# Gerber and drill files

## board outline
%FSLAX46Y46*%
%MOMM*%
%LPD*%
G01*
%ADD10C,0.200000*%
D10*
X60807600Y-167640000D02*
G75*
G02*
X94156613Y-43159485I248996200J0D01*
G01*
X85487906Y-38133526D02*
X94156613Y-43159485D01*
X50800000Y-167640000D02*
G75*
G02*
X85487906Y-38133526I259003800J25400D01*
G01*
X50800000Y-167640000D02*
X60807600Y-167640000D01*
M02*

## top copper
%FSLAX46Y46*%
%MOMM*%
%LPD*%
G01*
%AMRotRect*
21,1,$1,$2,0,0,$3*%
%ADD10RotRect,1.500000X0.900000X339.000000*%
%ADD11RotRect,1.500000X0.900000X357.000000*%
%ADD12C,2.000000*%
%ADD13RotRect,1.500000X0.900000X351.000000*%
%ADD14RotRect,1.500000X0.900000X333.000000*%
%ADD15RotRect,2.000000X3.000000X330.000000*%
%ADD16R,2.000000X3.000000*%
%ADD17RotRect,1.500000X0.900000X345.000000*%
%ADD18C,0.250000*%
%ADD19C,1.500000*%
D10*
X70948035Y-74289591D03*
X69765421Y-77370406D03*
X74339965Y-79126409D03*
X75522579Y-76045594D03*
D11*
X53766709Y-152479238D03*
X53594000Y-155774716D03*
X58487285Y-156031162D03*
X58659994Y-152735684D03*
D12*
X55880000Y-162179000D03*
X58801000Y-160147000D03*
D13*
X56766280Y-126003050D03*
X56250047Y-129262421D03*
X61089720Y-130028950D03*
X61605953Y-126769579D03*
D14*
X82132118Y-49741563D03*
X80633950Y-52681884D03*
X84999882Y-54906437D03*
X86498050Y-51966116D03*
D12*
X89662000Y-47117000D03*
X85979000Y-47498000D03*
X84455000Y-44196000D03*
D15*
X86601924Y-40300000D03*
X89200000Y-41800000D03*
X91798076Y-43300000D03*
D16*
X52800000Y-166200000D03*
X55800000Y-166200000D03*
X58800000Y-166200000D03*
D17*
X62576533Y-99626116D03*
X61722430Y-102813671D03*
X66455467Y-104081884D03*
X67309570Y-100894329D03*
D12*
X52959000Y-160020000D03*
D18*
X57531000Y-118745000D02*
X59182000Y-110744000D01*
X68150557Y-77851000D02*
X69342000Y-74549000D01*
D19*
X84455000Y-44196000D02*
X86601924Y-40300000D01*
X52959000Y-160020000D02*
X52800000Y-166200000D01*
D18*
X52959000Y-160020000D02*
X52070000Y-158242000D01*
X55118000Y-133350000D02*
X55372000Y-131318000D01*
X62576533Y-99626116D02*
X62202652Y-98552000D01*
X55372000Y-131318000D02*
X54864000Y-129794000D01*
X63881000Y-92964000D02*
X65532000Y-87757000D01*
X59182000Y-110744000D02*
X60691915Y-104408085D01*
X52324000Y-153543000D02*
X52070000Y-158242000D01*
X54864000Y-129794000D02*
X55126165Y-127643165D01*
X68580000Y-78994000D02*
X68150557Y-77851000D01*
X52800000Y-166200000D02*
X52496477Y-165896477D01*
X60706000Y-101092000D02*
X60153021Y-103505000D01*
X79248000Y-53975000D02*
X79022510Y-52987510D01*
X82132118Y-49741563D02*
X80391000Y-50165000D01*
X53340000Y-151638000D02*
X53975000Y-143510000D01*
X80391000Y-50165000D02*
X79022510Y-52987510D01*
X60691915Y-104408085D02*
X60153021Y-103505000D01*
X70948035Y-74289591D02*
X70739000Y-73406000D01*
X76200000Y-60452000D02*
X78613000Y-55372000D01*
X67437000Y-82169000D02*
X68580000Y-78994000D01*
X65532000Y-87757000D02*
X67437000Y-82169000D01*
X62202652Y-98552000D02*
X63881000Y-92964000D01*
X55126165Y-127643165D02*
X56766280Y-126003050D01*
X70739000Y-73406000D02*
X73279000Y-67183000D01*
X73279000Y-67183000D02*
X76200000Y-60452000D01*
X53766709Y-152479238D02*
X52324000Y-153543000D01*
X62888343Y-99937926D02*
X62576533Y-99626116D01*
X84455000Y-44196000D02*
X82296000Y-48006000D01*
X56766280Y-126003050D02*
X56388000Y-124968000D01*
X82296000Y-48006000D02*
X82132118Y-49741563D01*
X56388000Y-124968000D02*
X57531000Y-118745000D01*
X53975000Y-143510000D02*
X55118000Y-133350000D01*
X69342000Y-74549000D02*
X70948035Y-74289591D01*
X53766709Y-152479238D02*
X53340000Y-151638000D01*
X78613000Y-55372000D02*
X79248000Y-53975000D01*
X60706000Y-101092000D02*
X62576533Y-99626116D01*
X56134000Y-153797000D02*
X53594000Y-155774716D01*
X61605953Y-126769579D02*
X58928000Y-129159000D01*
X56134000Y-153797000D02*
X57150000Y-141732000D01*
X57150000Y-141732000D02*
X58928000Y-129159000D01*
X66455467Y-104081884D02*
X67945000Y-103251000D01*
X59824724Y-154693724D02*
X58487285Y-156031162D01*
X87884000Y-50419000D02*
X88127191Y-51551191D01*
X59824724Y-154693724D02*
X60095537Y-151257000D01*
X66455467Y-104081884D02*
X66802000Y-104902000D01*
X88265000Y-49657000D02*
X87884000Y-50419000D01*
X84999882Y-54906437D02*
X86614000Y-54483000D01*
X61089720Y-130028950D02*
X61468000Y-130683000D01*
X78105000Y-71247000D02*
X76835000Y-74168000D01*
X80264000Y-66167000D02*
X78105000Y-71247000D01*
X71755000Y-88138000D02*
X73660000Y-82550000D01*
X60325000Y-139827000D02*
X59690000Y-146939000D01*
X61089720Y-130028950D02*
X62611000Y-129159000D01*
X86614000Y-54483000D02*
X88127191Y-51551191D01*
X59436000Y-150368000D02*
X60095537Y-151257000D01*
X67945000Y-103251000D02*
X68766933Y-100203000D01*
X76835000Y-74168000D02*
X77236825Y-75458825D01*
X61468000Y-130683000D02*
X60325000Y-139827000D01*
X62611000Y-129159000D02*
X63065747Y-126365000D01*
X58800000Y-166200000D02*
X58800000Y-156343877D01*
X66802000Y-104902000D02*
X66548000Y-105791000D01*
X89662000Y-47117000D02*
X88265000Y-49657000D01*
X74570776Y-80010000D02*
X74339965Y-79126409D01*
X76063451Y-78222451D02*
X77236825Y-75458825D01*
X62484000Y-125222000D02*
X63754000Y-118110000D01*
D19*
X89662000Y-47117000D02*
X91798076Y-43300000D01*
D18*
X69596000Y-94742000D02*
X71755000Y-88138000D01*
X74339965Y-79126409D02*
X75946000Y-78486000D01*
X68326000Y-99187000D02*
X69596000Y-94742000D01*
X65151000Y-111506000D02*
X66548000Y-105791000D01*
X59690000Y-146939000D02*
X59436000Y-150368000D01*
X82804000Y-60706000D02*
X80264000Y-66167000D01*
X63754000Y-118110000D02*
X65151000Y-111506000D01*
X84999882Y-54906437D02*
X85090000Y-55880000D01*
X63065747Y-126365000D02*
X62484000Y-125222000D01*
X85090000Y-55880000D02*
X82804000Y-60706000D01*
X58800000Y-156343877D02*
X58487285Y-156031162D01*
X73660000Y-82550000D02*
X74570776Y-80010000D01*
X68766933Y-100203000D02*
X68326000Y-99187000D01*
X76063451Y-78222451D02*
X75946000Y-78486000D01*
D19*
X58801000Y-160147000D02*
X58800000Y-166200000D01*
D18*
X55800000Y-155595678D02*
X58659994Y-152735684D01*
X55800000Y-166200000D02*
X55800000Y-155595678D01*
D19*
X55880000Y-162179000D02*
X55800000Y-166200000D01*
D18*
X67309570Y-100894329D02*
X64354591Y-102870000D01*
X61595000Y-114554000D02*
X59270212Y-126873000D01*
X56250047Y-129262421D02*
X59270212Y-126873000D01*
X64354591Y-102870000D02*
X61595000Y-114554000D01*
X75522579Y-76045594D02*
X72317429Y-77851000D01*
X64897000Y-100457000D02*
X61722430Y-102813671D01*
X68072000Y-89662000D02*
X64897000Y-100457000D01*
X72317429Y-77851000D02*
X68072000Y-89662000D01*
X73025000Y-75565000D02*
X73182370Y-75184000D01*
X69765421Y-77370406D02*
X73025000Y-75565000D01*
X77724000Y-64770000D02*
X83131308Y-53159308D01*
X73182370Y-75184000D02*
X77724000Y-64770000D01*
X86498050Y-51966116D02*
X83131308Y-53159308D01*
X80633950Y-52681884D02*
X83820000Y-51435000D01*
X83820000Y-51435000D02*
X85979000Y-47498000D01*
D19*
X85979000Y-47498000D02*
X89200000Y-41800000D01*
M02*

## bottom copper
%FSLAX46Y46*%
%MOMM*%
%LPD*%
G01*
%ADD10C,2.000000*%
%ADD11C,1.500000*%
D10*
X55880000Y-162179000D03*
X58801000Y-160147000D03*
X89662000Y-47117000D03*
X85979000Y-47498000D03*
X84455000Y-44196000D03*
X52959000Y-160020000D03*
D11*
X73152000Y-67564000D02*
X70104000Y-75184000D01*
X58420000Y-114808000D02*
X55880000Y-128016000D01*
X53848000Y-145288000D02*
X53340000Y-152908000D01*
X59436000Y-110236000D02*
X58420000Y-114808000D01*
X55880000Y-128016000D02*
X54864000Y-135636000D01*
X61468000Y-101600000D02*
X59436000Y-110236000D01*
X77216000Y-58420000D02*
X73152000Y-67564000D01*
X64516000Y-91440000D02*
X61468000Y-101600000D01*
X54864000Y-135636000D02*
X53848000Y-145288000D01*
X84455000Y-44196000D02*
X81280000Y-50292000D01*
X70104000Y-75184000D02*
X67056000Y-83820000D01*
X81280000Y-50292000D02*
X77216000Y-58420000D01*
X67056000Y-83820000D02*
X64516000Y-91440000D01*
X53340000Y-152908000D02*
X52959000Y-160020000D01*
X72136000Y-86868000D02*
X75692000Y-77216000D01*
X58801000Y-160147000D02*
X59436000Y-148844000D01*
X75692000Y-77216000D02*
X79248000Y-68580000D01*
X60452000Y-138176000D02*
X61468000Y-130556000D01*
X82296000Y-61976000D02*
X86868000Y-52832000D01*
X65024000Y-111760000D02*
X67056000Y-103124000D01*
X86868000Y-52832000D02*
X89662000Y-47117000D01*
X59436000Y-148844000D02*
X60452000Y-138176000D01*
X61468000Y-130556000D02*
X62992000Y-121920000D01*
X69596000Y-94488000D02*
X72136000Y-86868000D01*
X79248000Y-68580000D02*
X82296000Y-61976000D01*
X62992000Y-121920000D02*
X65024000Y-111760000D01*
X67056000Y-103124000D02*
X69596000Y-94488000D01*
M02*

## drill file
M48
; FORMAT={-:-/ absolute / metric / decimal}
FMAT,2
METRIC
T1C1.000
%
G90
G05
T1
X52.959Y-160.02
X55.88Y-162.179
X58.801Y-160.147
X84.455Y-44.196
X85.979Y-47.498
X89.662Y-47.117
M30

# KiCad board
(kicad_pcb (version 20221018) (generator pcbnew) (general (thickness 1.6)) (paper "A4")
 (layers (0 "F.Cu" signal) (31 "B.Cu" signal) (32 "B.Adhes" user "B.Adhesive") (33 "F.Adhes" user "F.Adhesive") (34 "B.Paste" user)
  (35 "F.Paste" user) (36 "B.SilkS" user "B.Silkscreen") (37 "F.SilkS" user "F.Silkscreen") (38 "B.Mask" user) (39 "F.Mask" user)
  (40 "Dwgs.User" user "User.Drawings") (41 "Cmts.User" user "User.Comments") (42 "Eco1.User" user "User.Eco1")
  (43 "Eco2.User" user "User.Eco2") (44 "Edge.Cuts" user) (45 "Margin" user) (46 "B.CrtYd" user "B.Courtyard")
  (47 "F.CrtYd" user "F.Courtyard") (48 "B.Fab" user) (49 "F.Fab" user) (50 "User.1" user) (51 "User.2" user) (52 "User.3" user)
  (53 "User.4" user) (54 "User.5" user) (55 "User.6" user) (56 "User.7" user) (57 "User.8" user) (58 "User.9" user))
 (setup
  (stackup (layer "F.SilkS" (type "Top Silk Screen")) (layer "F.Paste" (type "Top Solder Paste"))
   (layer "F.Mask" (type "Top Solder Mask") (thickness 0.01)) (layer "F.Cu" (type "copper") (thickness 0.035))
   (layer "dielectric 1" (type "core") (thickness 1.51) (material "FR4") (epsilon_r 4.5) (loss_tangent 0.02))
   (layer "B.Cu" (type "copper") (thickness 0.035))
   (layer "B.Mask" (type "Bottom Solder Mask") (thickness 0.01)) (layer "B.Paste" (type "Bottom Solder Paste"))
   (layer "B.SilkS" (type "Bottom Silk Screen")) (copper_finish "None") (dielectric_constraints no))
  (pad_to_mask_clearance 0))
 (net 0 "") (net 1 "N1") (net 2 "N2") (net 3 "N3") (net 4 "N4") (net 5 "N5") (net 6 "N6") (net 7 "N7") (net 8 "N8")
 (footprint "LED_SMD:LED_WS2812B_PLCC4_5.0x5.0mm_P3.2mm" (layer "F.Cu") (at 72.644 76.708 -21)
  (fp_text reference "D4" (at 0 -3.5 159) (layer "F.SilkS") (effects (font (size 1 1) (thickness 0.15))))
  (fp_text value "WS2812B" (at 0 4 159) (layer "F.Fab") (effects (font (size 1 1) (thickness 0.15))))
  (pad "1" smd rect (at -2.45 -1.65 339) (size 1.5 0.9) (layers "F.Cu" "F.Paste" "F.Mask") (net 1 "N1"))
  (pad "2" smd rect (at -2.45 1.65 339) (size 1.5 0.9) (layers "F.Cu" "F.Paste" "F.Mask") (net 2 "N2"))
  (pad "3" smd rect (at 2.45 1.65 339) (size 1.5 0.9) (layers "F.Cu" "F.Paste" "F.Mask") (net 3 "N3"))
  (pad "4" smd rect (at 2.45 -1.65 339) (size 1.5 0.9) (layers "F.Cu" "F.Paste" "F.Mask") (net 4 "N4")))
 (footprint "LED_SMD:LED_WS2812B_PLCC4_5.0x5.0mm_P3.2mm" (layer "F.Cu") (at 56.126997 154.2552 -3)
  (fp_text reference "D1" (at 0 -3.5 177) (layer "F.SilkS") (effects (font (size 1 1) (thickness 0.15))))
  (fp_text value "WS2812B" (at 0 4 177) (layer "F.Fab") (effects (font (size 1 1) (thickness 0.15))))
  (pad "1" smd rect (at -2.45 -1.65 357) (size 1.5 0.9) (layers "F.Cu" "F.Paste" "F.Mask") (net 1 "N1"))
  (pad "2" smd rect (at -2.45 1.65 357) (size 1.5 0.9) (layers "F.Cu" "F.Paste" "F.Mask") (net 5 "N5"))
  (pad "3" smd rect (at 2.45 1.65 357) (size 1.5 0.9) (layers "F.Cu" "F.Paste" "F.Mask") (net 3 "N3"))
  (pad "4" smd rect (at 2.45 -1.65 357) (size 1.5 0.9) (layers "F.Cu" "F.Paste" "F.Mask") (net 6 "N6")))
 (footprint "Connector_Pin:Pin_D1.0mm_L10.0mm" (layer "F.Cu") (at 55.88 162.179 -4.5)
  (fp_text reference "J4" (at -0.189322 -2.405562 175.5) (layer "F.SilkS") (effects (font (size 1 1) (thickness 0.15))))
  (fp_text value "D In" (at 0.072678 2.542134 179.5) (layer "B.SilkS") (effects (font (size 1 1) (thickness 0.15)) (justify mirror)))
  (pad "1" thru_hole circle (at 0 0 355.5) (size 2 2) (drill 1) (layers "*.Cu" "*.Mask") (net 6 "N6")))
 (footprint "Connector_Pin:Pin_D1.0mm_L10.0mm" (layer "F.Cu") (at 58.801 160.147 -4.5)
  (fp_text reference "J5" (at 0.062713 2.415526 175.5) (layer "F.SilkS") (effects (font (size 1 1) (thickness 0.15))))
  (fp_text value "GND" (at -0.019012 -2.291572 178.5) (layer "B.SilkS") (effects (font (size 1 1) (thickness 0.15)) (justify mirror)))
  (pad "1" thru_hole circle (at 0 0 355.5) (size 2 2) (drill 1) (layers "*.Cu" "*.Mask") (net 3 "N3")))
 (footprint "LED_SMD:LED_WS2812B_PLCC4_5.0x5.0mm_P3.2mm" (layer "F.Cu") (at 58.928 128.016 -9)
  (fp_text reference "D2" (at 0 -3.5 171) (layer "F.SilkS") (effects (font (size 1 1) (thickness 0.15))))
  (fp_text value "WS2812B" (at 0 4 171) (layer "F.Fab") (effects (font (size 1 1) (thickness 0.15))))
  (pad "1" smd rect (at -2.45 -1.65 351) (size 1.5 0.9) (layers "F.Cu" "F.Paste" "F.Mask") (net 1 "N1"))
  (pad "2" smd rect (at -2.45 1.65 351) (size 1.5 0.9) (layers "F.Cu" "F.Paste" "F.Mask") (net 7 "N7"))
  (pad "3" smd rect (at 2.45 1.65 351) (size 1.5 0.9) (layers "F.Cu" "F.Paste" "F.Mask") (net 3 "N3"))
  (pad "4" smd rect (at 2.45 -1.65 351) (size 1.5 0.9) (layers "F.Cu" "F.Paste" "F.Mask") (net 5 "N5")))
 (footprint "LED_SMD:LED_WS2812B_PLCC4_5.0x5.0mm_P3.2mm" (layer "F.Cu") (at 83.566 52.324 -27)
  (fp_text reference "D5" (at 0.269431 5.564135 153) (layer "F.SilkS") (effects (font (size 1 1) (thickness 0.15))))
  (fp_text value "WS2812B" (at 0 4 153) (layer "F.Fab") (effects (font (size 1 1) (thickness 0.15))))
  (pad "1" smd rect (at -2.45 -1.65 333) (size 1.5 0.9) (layers "F.Cu" "F.Paste" "F.Mask") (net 1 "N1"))
  (pad "2" smd rect (at -2.45 1.65 333) (size 1.5 0.9) (layers "F.Cu" "F.Paste" "F.Mask") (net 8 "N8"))
  (pad "3" smd rect (at 2.45 1.65 333) (size 1.5 0.9) (layers "F.Cu" "F.Paste" "F.Mask") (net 3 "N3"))
  (pad "4" smd rect (at 2.45 -1.65 333) (size 1.5 0.9) (layers "F.Cu" "F.Paste" "F.Mask") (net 2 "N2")))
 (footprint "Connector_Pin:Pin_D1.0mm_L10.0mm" (layer "F.Cu") (at 89.662 47.117 -28)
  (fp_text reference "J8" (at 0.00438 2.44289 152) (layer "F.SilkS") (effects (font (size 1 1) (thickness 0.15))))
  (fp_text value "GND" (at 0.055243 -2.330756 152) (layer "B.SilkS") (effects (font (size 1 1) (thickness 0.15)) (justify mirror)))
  (pad "1" thru_hole circle (at 0 0 332) (size 2 2) (drill 1) (layers "*.Cu" "*.Mask") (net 3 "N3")))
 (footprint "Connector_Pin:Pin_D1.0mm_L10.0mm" (layer "F.Cu") (at 85.979 47.498 -25)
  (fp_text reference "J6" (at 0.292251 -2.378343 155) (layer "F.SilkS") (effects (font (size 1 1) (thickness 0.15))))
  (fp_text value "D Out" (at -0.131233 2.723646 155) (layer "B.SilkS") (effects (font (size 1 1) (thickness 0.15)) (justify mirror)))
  (pad "1" thru_hole circle (at 0 0 335) (size 2 2) (drill 1) (layers "*.Cu" "*.Mask") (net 8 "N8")))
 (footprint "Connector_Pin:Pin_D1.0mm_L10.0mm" (layer "F.Cu") (at 84.455 44.196 -25)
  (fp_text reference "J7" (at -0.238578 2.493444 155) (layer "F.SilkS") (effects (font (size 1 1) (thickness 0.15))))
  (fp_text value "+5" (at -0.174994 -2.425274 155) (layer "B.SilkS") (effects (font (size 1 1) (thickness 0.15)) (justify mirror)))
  (pad "1" thru_hole circle (at 0 0 335) (size 2 2) (drill 1) (layers "*.Cu" "*.Mask") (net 1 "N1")))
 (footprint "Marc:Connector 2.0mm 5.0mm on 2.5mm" (layer "F.Cu") (at 89.2 41.8 -30)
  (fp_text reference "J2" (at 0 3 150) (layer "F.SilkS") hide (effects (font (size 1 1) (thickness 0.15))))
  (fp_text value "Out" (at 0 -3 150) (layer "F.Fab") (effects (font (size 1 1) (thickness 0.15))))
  (pad "1" connect rect (at -3 0 330) (size 2 3) (layers "F.Cu" "F.Mask") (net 1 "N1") (thermal_bridge_angle 45))
  (pad "2" connect rect (at 0 0 330) (size 2 3) (layers "F.Cu" "F.Mask") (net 8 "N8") (thermal_bridge_angle 45))
  (pad "3" connect rect (at 3 0 330) (size 2 3) (layers "F.Cu" "F.Mask") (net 3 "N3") (thermal_bridge_angle 45)))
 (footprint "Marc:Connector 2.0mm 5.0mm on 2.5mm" (layer "F.Cu") (at 55.8 166.2)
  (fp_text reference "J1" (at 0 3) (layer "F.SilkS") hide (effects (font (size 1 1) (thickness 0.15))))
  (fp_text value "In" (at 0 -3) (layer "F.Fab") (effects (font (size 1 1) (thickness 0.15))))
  (pad "1" connect rect (at -3 0) (size 2 3) (layers "F.Cu" "F.Mask") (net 1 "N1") (thermal_bridge_angle 45))
  (pad "2" connect rect (at 0 0) (size 2 3) (layers "F.Cu" "F.Mask") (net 6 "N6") (thermal_bridge_angle 45))
  (pad "3" connect rect (at 3 0) (size 2 3) (layers "F.Cu" "F.Mask") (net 3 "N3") (thermal_bridge_angle 45)))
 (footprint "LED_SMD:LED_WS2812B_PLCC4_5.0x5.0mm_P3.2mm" (layer "F.Cu") (at 64.516 101.854 -15)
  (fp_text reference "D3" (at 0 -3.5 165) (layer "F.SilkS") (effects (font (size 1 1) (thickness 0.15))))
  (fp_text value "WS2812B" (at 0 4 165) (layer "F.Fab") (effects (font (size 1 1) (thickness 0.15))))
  (pad "1" smd rect (at -2.45 -1.65 345) (size 1.5 0.9) (layers "F.Cu" "F.Paste" "F.Mask") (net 1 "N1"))
  (pad "2" smd rect (at -2.45 1.65 345) (size 1.5 0.9) (layers "F.Cu" "F.Paste" "F.Mask") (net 4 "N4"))
  (pad "3" smd rect (at 2.45 1.65 345) (size 1.5 0.9) (layers "F.Cu" "F.Paste" "F.Mask") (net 3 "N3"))
  (pad "4" smd rect (at 2.45 -1.65 345) (size 1.5 0.9) (layers "F.Cu" "F.Paste" "F.Mask") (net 7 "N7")))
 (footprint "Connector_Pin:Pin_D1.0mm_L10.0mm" (layer "F.Cu") (at 52.959 160.02 -4.5)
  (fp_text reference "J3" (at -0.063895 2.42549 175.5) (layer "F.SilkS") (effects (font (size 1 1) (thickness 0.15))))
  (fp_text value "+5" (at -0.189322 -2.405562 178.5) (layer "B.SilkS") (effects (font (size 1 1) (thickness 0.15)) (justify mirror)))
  (pad "1" thru_hole circle (at 0 0 355.5) (size 2 2) (drill 1) (layers "*.Cu" "*.Mask") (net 1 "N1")))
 (gr_arc (start 60.8076 167.64) (mid 69.289312 103.204848) (end 94.156613 43.159485) (stroke (width 0.2) (type default)) (layer "Edge.Cuts"))
 (gr_line (start 85.487906 38.133526) (end 94.156613 43.159485) (stroke (width 0.2) (type default)) (layer "Edge.Cuts"))
 (gr_arc (start 50.8 167.64) (mid 59.618942 100.603365) (end 85.487906 38.133526) (stroke (width 0.2) (type default)) (layer "Edge.Cuts"))
 (gr_line (start 50.8 167.64) (end 60.8076 167.64) (stroke (width 0.2) (type default)) (layer "Edge.Cuts"))
 (segment (start 57.531 118.745) (end 59.182 110.744) (width 0.25) (layer "F.Cu") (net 1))
 (segment (start 68.150557 77.851) (end 69.342 74.549) (width 0.25) (layer "F.Cu") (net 1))
 (segment (start 84.455 44.196) (end 86.601924 40.3) (width 1.5) (layer "F.Cu") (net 1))
 (segment (start 52.959 160.02) (end 52.8 166.2) (width 1.5) (layer "F.Cu") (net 1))
 (segment (start 52.959 160.02) (end 52.07 158.242) (width 0.25) (layer "F.Cu") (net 1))
 (segment (start 55.118 133.35) (end 55.372 131.318) (width 0.25) (layer "F.Cu") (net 1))
 (segment (start 62.576533 99.626116) (end 62.202652 98.552) (width 0.25) (layer "F.Cu") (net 1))
 (segment (start 55.372 131.318) (end 54.864 129.794) (width 0.25) (layer "F.Cu") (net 1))
 (segment (start 63.881 92.964) (end 65.532 87.757) (width 0.25) (layer "F.Cu") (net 1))
 (segment (start 59.182 110.744) (end 60.691915 104.408085) (width 0.25) (layer "F.Cu") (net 1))
 (segment (start 52.324 153.543) (end 52.07 158.242) (width 0.25) (layer "F.Cu") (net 1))
 (segment (start 54.864 129.794) (end 55.126165 127.643165) (width 0.25) (layer "F.Cu") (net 1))
 (segment (start 68.58 78.994) (end 68.150557 77.851) (width 0.25) (layer "F.Cu") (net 1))
 (segment (start 52.8 166.2) (end 52.496477 165.896477) (width 0.25) (layer "F.Cu") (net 1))
 (segment (start 60.706 101.092) (end 60.153021 103.505) (width 0.25) (layer "F.Cu") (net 1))
 (segment (start 79.248 53.975) (end 79.02251 52.98751) (width 0.25) (layer "F.Cu") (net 1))
 (segment (start 82.132118 49.741563) (end 80.391 50.165) (width 0.25) (layer "F.Cu") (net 1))
 (segment (start 53.34 151.638) (end 53.975 143.51) (width 0.25) (layer "F.Cu") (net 1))
 (segment (start 80.391 50.165) (end 79.02251 52.98751) (width 0.25) (layer "F.Cu") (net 1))
 (segment (start 60.691915 104.408085) (end 60.153021 103.505) (width 0.25) (layer "F.Cu") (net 1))
 (segment (start 70.948035 74.289591) (end 70.739 73.406) (width 0.25) (layer "F.Cu") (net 1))
 (segment (start 76.2 60.452) (end 78.613 55.372) (width 0.25) (layer "F.Cu") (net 1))
 (segment (start 67.437 82.169) (end 68.58 78.994) (width 0.25) (layer "F.Cu") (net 1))
 (segment (start 65.532 87.757) (end 67.437 82.169) (width 0.25) (layer "F.Cu") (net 1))
 (segment (start 62.202652 98.552) (end 63.881 92.964) (width 0.25) (layer "F.Cu") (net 1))
 (segment (start 55.126165 127.643165) (end 56.76628 126.00305) (width 0.25) (layer "F.Cu") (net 1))
 (segment (start 70.739 73.406) (end 73.279 67.183) (width 0.25) (layer "F.Cu") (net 1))
 (segment (start 73.279 67.183) (end 76.2 60.452) (width 0.25) (layer "F.Cu") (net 1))
 (segment (start 53.766709 152.479238) (end 52.324 153.543) (width 0.25) (layer "F.Cu") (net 1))
 (segment (start 62.888343 99.937926) (end 62.576533 99.626116) (width 0.25) (layer "F.Cu") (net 1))
 (segment (start 84.455 44.196) (end 82.296 48.006) (width 0.25) (layer "F.Cu") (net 1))
 (segment (start 56.76628 126.00305) (end 56.388 124.968) (width 0.25) (layer "F.Cu") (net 1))
 (segment (start 82.296 48.006) (end 82.132118 49.741563) (width 0.25) (layer "F.Cu") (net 1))
 (segment (start 56.388 124.968) (end 57.531 118.745) (width 0.25) (layer "F.Cu") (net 1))
 (segment (start 53.975 143.51) (end 55.118 133.35) (width 0.25) (layer "F.Cu") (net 1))
 (segment (start 69.342 74.549) (end 70.948035 74.289591) (width 0.25) (layer "F.Cu") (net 1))
 (segment (start 53.766709 152.479238) (end 53.34 151.638) (width 0.25) (layer "F.Cu") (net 1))
 (segment (start 78.613 55.372) (end 79.248 53.975) (width 0.25) (layer "F.Cu") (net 1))
 (segment (start 60.706 101.092) (end 62.576533 99.626116) (width 0.25) (layer "F.Cu") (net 1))
 (segment (start 73.152 67.564) (end 70.104 75.184) (width 1.5) (layer "B.Cu") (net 1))
 (segment (start 58.42 114.808) (end 55.88 128.016) (width 1.5) (layer "B.Cu") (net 1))
 (segment (start 53.848 145.288) (end 53.34 152.908) (width 1.5) (layer "B.Cu") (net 1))
 (segment (start 59.436 110.236) (end 58.42 114.808) (width 1.5) (layer "B.Cu") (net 1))
 (segment (start 55.88 128.016) (end 54.864 135.636) (width 1.5) (layer "B.Cu") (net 1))
 (segment (start 61.468 101.6) (end 59.436 110.236) (width 1.5) (layer "B.Cu") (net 1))
 (segment (start 77.216 58.42) (end 73.152 67.564) (width 1.5) (layer "B.Cu") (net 1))
 (segment (start 64.516 91.44) (end 61.468 101.6) (width 1.5) (layer "B.Cu") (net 1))
 (segment (start 54.864 135.636) (end 53.848 145.288) (width 1.5) (layer "B.Cu") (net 1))
 (segment (start 84.455 44.196) (end 81.28 50.292) (width 1.5) (layer "B.Cu") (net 1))
 (segment (start 70.104 75.184) (end 67.056 83.82) (width 1.5) (layer "B.Cu") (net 1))
 (segment (start 81.28 50.292) (end 77.216 58.42) (width 1.5) (layer "B.Cu") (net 1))
 (segment (start 67.056 83.82) (end 64.516 91.44) (width 1.5) (layer "B.Cu") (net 1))
 (segment (start 53.34 152.908) (end 52.959 160.02) (width 1.5) (layer "B.Cu") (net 1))
 (segment (start 56.134 153.797) (end 53.594 155.774716) (width 0.25) (layer "F.Cu") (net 5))
 (segment (start 61.605953 126.769579) (end 58.928 129.159) (width 0.25) (layer "F.Cu") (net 5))
 (segment (start 56.134 153.797) (end 57.15 141.732) (width 0.25) (layer "F.Cu") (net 5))
 (segment (start 57.15 141.732) (end 58.928 129.159) (width 0.25) (layer "F.Cu") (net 5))
 (segment (start 66.455467 104.081884) (end 67.945 103.251) (width 0.25) (layer "F.Cu") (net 3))
 (segment (start 59.824724 154.693724) (end 58.487285 156.031162) (width 0.25) (layer "F.Cu") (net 3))
 (segment (start 87.884 50.419) (end 88.127191 51.551191) (width 0.25) (layer "F.Cu") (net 3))
 (segment (start 59.824724 154.693724) (end 60.095537 151.257) (width 0.25) (layer "F.Cu") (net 3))
 (segment (start 66.455467 104.081884) (end 66.802 104.902) (width 0.25) (layer "F.Cu") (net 3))
 (segment (start 88.265 49.657) (end 87.884 50.419) (width 0.25) (layer "F.Cu") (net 3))
 (segment (start 84.999882 54.906437) (end 86.614 54.483) (width 0.25) (layer "F.Cu") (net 3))
 (segment (start 61.08972 130.02895) (end 61.468 130.683) (width 0.25) (layer "F.Cu") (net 3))
 (segment (start 78.105 71.247) (end 76.835 74.168) (width 0.25) (layer "F.Cu") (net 3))
 (segment (start 80.264 66.167) (end 78.105 71.247) (width 0.25) (layer "F.Cu") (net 3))
 (segment (start 71.755 88.138) (end 73.66 82.55) (width 0.25) (layer "F.Cu") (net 3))
 (segment (start 60.325 139.827) (end 59.69 146.939) (width 0.25) (layer "F.Cu") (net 3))
 (segment (start 61.08972 130.02895) (end 62.611 129.159) (width 0.25) (layer "F.Cu") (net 3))
 (segment (start 86.614 54.483) (end 88.127191 51.551191) (width 0.25) (layer "F.Cu") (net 3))
 (segment (start 59.436 150.368) (end 60.095537 151.257) (width 0.25) (layer "F.Cu") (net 3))
 (segment (start 67.945 103.251) (end 68.766933 100.203) (width 0.25) (layer "F.Cu") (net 3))
 (segment (start 76.835 74.168) (end 77.236825 75.458825) (width 0.25) (layer "F.Cu") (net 3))
 (segment (start 61.468 130.683) (end 60.325 139.827) (width 0.25) (layer "F.Cu") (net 3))
 (segment (start 62.611 129.159) (end 63.065747 126.365) (width 0.25) (layer "F.Cu") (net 3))
 (segment (start 58.8 166.2) (end 58.8 156.343877) (width 0.25) (layer "F.Cu") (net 3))
 (segment (start 66.802 104.902) (end 66.548 105.791) (width 0.25) (layer "F.Cu") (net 3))
 (segment (start 89.662 47.117) (end 88.265 49.657) (width 0.25) (layer "F.Cu") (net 3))
 (segment (start 74.570776 80.01) (end 74.339965 79.126409) (width 0.25) (layer "F.Cu") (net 3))
 (segment (start 76.063451 78.222451) (end 77.236825 75.458825) (width 0.25) (layer "F.Cu") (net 3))
 (segment (start 62.484 125.222) (end 63.754 118.11) (width 0.25) (layer "F.Cu") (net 3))
 (segment (start 89.662 47.117) (end 91.798076 43.3) (width 1.5) (layer "F.Cu") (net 3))
 (segment (start 69.596 94.742) (end 71.755 88.138) (width 0.25) (layer "F.Cu") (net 3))
 (segment (start 74.339965 79.126409) (end 75.946 78.486) (width 0.25) (layer "F.Cu") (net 3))
 (segment (start 68.326 99.187) (end 69.596 94.742) (width 0.25) (layer "F.Cu") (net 3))
 (segment (start 65.151 111.506) (end 66.548 105.791) (width 0.25) (layer "F.Cu") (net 3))
 (segment (start 59.69 146.939) (end 59.436 150.368) (width 0.25) (layer "F.Cu") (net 3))
 (segment (start 82.804 60.706) (end 80.264 66.167) (width 0.25) (layer "F.Cu") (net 3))
 (segment (start 63.754 118.11) (end 65.151 111.506) (width 0.25) (layer "F.Cu") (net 3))
 (segment (start 84.999882 54.906437) (end 85.09 55.88) (width 0.25) (layer "F.Cu") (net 3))
 (segment (start 63.065747 126.365) (end 62.484 125.222) (width 0.25) (layer "F.Cu") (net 3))
 (segment (start 85.09 55.88) (end 82.804 60.706) (width 0.25) (layer "F.Cu") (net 3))
 (segment (start 58.8 156.343877) (end 58.487285 156.031162) (width 0.25) (layer "F.Cu") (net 3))
 (segment (start 73.66 82.55) (end 74.570776 80.01) (width 0.25) (layer "F.Cu") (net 3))
 (segment (start 68.766933 100.203) (end 68.326 99.187) (width 0.25) (layer "F.Cu") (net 3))
 (segment (start 76.063451 78.222451) (end 75.946 78.486) (width 0.25) (layer "F.Cu") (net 3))
 (segment (start 58.801 160.147) (end 58.8 166.2) (width 1.5) (layer "F.Cu") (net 3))
 (segment (start 72.136 86.868) (end 75.692 77.216) (width 1.5) (layer "B.Cu") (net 3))
 (segment (start 58.801 160.147) (end 59.436 148.844) (width 1.5) (layer "B.Cu") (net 3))
 (segment (start 75.692 77.216) (end 79.248 68.58) (width 1.5) (layer "B.Cu") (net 3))
 (segment (start 60.452 138.176) (end 61.468 130.556) (width 1.5) (layer "B.Cu") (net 3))
 (segment (start 82.296 61.976) (end 86.868 52.832) (width 1.5) (layer "B.Cu") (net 3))
 (segment (start 65.024 111.76) (end 67.056 103.124) (width 1.5) (layer "B.Cu") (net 3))
 (segment (start 86.868 52.832) (end 89.662 47.117) (width 1.5) (layer "B.Cu") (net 3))
 (segment (start 59.436 148.844) (end 60.452 138.176) (width 1.5) (layer "B.Cu") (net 3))
 (segment (start 61.468 130.556) (end 62.992 121.92) (width 1.5) (layer "B.Cu") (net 3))
 (segment (start 69.596 94.488) (end 72.136 86.868) (width 1.5) (layer "B.Cu") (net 3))
 (segment (start 79.248 68.58) (end 82.296 61.976) (width 1.5) (layer "B.Cu") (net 3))
 (segment (start 62.992 121.92) (end 65.024 111.76) (width 1.5) (layer "B.Cu") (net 3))
 (segment (start 67.056 103.124) (end 69.596 94.488) (width 1.5) (layer "B.Cu") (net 3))
 (segment (start 55.8 155.595678) (end 58.659994 152.735684) (width 0.25) (layer "F.Cu") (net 6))
 (segment (start 55.8 166.2) (end 55.8 155.595678) (width 0.25) (layer "F.Cu") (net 6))
 (segment (start 55.88 162.179) (end 55.8 166.2) (width 1.5) (layer "F.Cu") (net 6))
 (segment (start 67.30957 100.894329) (end 64.354591 102.87) (width 0.25) (layer "F.Cu") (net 7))
 (segment (start 61.595 114.554) (end 59.270212 126.873) (width 0.25) (layer "F.Cu") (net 7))
 (segment (start 56.250047 129.262421) (end 59.270212 126.873) (width 0.25) (layer "F.Cu") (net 7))
 (segment (start 64.354591 102.87) (end 61.595 114.554) (width 0.25) (layer "F.Cu") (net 7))
 (segment (start 75.522579 76.045594) (end 72.317429 77.851) (width 0.25) (layer "F.Cu") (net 4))
 (segment (start 64.897 100.457) (end 61.72243 102.813671) (width 0.25) (layer "F.Cu") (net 4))
 (segment (start 68.072 89.662) (end 64.897 100.457) (width 0.25) (layer "F.Cu") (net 4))
 (segment (start 72.317429 77.851) (end 68.072 89.662) (width 0.25) (layer "F.Cu") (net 4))
 (segment (start 73.025 75.565) (end 73.18237 75.184) (width 0.25) (layer "F.Cu") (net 2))
 (segment (start 69.765421 77.370406) (end 73.025 75.565) (width 0.25) (layer "F.Cu") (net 2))
 (segment (start 77.724 64.77) (end 83.131308 53.159308) (width 0.25) (layer "F.Cu") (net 2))
 (segment (start 73.18237 75.184) (end 77.724 64.77) (width 0.25) (layer "F.Cu") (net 2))
 (segment (start 86.49805 51.966116) (end 83.131308 53.159308) (width 0.25) (layer "F.Cu") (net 2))
 (segment (start 80.63395 52.681884) (end 83.82 51.435) (width 0.25) (layer "F.Cu") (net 8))
 (segment (start 83.82 51.435) (end 85.979 47.498) (width 0.25) (layer "F.Cu") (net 8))
 (segment (start 85.979 47.498) (end 89.2 41.8) (width 1.5) (layer "F.Cu") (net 8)))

